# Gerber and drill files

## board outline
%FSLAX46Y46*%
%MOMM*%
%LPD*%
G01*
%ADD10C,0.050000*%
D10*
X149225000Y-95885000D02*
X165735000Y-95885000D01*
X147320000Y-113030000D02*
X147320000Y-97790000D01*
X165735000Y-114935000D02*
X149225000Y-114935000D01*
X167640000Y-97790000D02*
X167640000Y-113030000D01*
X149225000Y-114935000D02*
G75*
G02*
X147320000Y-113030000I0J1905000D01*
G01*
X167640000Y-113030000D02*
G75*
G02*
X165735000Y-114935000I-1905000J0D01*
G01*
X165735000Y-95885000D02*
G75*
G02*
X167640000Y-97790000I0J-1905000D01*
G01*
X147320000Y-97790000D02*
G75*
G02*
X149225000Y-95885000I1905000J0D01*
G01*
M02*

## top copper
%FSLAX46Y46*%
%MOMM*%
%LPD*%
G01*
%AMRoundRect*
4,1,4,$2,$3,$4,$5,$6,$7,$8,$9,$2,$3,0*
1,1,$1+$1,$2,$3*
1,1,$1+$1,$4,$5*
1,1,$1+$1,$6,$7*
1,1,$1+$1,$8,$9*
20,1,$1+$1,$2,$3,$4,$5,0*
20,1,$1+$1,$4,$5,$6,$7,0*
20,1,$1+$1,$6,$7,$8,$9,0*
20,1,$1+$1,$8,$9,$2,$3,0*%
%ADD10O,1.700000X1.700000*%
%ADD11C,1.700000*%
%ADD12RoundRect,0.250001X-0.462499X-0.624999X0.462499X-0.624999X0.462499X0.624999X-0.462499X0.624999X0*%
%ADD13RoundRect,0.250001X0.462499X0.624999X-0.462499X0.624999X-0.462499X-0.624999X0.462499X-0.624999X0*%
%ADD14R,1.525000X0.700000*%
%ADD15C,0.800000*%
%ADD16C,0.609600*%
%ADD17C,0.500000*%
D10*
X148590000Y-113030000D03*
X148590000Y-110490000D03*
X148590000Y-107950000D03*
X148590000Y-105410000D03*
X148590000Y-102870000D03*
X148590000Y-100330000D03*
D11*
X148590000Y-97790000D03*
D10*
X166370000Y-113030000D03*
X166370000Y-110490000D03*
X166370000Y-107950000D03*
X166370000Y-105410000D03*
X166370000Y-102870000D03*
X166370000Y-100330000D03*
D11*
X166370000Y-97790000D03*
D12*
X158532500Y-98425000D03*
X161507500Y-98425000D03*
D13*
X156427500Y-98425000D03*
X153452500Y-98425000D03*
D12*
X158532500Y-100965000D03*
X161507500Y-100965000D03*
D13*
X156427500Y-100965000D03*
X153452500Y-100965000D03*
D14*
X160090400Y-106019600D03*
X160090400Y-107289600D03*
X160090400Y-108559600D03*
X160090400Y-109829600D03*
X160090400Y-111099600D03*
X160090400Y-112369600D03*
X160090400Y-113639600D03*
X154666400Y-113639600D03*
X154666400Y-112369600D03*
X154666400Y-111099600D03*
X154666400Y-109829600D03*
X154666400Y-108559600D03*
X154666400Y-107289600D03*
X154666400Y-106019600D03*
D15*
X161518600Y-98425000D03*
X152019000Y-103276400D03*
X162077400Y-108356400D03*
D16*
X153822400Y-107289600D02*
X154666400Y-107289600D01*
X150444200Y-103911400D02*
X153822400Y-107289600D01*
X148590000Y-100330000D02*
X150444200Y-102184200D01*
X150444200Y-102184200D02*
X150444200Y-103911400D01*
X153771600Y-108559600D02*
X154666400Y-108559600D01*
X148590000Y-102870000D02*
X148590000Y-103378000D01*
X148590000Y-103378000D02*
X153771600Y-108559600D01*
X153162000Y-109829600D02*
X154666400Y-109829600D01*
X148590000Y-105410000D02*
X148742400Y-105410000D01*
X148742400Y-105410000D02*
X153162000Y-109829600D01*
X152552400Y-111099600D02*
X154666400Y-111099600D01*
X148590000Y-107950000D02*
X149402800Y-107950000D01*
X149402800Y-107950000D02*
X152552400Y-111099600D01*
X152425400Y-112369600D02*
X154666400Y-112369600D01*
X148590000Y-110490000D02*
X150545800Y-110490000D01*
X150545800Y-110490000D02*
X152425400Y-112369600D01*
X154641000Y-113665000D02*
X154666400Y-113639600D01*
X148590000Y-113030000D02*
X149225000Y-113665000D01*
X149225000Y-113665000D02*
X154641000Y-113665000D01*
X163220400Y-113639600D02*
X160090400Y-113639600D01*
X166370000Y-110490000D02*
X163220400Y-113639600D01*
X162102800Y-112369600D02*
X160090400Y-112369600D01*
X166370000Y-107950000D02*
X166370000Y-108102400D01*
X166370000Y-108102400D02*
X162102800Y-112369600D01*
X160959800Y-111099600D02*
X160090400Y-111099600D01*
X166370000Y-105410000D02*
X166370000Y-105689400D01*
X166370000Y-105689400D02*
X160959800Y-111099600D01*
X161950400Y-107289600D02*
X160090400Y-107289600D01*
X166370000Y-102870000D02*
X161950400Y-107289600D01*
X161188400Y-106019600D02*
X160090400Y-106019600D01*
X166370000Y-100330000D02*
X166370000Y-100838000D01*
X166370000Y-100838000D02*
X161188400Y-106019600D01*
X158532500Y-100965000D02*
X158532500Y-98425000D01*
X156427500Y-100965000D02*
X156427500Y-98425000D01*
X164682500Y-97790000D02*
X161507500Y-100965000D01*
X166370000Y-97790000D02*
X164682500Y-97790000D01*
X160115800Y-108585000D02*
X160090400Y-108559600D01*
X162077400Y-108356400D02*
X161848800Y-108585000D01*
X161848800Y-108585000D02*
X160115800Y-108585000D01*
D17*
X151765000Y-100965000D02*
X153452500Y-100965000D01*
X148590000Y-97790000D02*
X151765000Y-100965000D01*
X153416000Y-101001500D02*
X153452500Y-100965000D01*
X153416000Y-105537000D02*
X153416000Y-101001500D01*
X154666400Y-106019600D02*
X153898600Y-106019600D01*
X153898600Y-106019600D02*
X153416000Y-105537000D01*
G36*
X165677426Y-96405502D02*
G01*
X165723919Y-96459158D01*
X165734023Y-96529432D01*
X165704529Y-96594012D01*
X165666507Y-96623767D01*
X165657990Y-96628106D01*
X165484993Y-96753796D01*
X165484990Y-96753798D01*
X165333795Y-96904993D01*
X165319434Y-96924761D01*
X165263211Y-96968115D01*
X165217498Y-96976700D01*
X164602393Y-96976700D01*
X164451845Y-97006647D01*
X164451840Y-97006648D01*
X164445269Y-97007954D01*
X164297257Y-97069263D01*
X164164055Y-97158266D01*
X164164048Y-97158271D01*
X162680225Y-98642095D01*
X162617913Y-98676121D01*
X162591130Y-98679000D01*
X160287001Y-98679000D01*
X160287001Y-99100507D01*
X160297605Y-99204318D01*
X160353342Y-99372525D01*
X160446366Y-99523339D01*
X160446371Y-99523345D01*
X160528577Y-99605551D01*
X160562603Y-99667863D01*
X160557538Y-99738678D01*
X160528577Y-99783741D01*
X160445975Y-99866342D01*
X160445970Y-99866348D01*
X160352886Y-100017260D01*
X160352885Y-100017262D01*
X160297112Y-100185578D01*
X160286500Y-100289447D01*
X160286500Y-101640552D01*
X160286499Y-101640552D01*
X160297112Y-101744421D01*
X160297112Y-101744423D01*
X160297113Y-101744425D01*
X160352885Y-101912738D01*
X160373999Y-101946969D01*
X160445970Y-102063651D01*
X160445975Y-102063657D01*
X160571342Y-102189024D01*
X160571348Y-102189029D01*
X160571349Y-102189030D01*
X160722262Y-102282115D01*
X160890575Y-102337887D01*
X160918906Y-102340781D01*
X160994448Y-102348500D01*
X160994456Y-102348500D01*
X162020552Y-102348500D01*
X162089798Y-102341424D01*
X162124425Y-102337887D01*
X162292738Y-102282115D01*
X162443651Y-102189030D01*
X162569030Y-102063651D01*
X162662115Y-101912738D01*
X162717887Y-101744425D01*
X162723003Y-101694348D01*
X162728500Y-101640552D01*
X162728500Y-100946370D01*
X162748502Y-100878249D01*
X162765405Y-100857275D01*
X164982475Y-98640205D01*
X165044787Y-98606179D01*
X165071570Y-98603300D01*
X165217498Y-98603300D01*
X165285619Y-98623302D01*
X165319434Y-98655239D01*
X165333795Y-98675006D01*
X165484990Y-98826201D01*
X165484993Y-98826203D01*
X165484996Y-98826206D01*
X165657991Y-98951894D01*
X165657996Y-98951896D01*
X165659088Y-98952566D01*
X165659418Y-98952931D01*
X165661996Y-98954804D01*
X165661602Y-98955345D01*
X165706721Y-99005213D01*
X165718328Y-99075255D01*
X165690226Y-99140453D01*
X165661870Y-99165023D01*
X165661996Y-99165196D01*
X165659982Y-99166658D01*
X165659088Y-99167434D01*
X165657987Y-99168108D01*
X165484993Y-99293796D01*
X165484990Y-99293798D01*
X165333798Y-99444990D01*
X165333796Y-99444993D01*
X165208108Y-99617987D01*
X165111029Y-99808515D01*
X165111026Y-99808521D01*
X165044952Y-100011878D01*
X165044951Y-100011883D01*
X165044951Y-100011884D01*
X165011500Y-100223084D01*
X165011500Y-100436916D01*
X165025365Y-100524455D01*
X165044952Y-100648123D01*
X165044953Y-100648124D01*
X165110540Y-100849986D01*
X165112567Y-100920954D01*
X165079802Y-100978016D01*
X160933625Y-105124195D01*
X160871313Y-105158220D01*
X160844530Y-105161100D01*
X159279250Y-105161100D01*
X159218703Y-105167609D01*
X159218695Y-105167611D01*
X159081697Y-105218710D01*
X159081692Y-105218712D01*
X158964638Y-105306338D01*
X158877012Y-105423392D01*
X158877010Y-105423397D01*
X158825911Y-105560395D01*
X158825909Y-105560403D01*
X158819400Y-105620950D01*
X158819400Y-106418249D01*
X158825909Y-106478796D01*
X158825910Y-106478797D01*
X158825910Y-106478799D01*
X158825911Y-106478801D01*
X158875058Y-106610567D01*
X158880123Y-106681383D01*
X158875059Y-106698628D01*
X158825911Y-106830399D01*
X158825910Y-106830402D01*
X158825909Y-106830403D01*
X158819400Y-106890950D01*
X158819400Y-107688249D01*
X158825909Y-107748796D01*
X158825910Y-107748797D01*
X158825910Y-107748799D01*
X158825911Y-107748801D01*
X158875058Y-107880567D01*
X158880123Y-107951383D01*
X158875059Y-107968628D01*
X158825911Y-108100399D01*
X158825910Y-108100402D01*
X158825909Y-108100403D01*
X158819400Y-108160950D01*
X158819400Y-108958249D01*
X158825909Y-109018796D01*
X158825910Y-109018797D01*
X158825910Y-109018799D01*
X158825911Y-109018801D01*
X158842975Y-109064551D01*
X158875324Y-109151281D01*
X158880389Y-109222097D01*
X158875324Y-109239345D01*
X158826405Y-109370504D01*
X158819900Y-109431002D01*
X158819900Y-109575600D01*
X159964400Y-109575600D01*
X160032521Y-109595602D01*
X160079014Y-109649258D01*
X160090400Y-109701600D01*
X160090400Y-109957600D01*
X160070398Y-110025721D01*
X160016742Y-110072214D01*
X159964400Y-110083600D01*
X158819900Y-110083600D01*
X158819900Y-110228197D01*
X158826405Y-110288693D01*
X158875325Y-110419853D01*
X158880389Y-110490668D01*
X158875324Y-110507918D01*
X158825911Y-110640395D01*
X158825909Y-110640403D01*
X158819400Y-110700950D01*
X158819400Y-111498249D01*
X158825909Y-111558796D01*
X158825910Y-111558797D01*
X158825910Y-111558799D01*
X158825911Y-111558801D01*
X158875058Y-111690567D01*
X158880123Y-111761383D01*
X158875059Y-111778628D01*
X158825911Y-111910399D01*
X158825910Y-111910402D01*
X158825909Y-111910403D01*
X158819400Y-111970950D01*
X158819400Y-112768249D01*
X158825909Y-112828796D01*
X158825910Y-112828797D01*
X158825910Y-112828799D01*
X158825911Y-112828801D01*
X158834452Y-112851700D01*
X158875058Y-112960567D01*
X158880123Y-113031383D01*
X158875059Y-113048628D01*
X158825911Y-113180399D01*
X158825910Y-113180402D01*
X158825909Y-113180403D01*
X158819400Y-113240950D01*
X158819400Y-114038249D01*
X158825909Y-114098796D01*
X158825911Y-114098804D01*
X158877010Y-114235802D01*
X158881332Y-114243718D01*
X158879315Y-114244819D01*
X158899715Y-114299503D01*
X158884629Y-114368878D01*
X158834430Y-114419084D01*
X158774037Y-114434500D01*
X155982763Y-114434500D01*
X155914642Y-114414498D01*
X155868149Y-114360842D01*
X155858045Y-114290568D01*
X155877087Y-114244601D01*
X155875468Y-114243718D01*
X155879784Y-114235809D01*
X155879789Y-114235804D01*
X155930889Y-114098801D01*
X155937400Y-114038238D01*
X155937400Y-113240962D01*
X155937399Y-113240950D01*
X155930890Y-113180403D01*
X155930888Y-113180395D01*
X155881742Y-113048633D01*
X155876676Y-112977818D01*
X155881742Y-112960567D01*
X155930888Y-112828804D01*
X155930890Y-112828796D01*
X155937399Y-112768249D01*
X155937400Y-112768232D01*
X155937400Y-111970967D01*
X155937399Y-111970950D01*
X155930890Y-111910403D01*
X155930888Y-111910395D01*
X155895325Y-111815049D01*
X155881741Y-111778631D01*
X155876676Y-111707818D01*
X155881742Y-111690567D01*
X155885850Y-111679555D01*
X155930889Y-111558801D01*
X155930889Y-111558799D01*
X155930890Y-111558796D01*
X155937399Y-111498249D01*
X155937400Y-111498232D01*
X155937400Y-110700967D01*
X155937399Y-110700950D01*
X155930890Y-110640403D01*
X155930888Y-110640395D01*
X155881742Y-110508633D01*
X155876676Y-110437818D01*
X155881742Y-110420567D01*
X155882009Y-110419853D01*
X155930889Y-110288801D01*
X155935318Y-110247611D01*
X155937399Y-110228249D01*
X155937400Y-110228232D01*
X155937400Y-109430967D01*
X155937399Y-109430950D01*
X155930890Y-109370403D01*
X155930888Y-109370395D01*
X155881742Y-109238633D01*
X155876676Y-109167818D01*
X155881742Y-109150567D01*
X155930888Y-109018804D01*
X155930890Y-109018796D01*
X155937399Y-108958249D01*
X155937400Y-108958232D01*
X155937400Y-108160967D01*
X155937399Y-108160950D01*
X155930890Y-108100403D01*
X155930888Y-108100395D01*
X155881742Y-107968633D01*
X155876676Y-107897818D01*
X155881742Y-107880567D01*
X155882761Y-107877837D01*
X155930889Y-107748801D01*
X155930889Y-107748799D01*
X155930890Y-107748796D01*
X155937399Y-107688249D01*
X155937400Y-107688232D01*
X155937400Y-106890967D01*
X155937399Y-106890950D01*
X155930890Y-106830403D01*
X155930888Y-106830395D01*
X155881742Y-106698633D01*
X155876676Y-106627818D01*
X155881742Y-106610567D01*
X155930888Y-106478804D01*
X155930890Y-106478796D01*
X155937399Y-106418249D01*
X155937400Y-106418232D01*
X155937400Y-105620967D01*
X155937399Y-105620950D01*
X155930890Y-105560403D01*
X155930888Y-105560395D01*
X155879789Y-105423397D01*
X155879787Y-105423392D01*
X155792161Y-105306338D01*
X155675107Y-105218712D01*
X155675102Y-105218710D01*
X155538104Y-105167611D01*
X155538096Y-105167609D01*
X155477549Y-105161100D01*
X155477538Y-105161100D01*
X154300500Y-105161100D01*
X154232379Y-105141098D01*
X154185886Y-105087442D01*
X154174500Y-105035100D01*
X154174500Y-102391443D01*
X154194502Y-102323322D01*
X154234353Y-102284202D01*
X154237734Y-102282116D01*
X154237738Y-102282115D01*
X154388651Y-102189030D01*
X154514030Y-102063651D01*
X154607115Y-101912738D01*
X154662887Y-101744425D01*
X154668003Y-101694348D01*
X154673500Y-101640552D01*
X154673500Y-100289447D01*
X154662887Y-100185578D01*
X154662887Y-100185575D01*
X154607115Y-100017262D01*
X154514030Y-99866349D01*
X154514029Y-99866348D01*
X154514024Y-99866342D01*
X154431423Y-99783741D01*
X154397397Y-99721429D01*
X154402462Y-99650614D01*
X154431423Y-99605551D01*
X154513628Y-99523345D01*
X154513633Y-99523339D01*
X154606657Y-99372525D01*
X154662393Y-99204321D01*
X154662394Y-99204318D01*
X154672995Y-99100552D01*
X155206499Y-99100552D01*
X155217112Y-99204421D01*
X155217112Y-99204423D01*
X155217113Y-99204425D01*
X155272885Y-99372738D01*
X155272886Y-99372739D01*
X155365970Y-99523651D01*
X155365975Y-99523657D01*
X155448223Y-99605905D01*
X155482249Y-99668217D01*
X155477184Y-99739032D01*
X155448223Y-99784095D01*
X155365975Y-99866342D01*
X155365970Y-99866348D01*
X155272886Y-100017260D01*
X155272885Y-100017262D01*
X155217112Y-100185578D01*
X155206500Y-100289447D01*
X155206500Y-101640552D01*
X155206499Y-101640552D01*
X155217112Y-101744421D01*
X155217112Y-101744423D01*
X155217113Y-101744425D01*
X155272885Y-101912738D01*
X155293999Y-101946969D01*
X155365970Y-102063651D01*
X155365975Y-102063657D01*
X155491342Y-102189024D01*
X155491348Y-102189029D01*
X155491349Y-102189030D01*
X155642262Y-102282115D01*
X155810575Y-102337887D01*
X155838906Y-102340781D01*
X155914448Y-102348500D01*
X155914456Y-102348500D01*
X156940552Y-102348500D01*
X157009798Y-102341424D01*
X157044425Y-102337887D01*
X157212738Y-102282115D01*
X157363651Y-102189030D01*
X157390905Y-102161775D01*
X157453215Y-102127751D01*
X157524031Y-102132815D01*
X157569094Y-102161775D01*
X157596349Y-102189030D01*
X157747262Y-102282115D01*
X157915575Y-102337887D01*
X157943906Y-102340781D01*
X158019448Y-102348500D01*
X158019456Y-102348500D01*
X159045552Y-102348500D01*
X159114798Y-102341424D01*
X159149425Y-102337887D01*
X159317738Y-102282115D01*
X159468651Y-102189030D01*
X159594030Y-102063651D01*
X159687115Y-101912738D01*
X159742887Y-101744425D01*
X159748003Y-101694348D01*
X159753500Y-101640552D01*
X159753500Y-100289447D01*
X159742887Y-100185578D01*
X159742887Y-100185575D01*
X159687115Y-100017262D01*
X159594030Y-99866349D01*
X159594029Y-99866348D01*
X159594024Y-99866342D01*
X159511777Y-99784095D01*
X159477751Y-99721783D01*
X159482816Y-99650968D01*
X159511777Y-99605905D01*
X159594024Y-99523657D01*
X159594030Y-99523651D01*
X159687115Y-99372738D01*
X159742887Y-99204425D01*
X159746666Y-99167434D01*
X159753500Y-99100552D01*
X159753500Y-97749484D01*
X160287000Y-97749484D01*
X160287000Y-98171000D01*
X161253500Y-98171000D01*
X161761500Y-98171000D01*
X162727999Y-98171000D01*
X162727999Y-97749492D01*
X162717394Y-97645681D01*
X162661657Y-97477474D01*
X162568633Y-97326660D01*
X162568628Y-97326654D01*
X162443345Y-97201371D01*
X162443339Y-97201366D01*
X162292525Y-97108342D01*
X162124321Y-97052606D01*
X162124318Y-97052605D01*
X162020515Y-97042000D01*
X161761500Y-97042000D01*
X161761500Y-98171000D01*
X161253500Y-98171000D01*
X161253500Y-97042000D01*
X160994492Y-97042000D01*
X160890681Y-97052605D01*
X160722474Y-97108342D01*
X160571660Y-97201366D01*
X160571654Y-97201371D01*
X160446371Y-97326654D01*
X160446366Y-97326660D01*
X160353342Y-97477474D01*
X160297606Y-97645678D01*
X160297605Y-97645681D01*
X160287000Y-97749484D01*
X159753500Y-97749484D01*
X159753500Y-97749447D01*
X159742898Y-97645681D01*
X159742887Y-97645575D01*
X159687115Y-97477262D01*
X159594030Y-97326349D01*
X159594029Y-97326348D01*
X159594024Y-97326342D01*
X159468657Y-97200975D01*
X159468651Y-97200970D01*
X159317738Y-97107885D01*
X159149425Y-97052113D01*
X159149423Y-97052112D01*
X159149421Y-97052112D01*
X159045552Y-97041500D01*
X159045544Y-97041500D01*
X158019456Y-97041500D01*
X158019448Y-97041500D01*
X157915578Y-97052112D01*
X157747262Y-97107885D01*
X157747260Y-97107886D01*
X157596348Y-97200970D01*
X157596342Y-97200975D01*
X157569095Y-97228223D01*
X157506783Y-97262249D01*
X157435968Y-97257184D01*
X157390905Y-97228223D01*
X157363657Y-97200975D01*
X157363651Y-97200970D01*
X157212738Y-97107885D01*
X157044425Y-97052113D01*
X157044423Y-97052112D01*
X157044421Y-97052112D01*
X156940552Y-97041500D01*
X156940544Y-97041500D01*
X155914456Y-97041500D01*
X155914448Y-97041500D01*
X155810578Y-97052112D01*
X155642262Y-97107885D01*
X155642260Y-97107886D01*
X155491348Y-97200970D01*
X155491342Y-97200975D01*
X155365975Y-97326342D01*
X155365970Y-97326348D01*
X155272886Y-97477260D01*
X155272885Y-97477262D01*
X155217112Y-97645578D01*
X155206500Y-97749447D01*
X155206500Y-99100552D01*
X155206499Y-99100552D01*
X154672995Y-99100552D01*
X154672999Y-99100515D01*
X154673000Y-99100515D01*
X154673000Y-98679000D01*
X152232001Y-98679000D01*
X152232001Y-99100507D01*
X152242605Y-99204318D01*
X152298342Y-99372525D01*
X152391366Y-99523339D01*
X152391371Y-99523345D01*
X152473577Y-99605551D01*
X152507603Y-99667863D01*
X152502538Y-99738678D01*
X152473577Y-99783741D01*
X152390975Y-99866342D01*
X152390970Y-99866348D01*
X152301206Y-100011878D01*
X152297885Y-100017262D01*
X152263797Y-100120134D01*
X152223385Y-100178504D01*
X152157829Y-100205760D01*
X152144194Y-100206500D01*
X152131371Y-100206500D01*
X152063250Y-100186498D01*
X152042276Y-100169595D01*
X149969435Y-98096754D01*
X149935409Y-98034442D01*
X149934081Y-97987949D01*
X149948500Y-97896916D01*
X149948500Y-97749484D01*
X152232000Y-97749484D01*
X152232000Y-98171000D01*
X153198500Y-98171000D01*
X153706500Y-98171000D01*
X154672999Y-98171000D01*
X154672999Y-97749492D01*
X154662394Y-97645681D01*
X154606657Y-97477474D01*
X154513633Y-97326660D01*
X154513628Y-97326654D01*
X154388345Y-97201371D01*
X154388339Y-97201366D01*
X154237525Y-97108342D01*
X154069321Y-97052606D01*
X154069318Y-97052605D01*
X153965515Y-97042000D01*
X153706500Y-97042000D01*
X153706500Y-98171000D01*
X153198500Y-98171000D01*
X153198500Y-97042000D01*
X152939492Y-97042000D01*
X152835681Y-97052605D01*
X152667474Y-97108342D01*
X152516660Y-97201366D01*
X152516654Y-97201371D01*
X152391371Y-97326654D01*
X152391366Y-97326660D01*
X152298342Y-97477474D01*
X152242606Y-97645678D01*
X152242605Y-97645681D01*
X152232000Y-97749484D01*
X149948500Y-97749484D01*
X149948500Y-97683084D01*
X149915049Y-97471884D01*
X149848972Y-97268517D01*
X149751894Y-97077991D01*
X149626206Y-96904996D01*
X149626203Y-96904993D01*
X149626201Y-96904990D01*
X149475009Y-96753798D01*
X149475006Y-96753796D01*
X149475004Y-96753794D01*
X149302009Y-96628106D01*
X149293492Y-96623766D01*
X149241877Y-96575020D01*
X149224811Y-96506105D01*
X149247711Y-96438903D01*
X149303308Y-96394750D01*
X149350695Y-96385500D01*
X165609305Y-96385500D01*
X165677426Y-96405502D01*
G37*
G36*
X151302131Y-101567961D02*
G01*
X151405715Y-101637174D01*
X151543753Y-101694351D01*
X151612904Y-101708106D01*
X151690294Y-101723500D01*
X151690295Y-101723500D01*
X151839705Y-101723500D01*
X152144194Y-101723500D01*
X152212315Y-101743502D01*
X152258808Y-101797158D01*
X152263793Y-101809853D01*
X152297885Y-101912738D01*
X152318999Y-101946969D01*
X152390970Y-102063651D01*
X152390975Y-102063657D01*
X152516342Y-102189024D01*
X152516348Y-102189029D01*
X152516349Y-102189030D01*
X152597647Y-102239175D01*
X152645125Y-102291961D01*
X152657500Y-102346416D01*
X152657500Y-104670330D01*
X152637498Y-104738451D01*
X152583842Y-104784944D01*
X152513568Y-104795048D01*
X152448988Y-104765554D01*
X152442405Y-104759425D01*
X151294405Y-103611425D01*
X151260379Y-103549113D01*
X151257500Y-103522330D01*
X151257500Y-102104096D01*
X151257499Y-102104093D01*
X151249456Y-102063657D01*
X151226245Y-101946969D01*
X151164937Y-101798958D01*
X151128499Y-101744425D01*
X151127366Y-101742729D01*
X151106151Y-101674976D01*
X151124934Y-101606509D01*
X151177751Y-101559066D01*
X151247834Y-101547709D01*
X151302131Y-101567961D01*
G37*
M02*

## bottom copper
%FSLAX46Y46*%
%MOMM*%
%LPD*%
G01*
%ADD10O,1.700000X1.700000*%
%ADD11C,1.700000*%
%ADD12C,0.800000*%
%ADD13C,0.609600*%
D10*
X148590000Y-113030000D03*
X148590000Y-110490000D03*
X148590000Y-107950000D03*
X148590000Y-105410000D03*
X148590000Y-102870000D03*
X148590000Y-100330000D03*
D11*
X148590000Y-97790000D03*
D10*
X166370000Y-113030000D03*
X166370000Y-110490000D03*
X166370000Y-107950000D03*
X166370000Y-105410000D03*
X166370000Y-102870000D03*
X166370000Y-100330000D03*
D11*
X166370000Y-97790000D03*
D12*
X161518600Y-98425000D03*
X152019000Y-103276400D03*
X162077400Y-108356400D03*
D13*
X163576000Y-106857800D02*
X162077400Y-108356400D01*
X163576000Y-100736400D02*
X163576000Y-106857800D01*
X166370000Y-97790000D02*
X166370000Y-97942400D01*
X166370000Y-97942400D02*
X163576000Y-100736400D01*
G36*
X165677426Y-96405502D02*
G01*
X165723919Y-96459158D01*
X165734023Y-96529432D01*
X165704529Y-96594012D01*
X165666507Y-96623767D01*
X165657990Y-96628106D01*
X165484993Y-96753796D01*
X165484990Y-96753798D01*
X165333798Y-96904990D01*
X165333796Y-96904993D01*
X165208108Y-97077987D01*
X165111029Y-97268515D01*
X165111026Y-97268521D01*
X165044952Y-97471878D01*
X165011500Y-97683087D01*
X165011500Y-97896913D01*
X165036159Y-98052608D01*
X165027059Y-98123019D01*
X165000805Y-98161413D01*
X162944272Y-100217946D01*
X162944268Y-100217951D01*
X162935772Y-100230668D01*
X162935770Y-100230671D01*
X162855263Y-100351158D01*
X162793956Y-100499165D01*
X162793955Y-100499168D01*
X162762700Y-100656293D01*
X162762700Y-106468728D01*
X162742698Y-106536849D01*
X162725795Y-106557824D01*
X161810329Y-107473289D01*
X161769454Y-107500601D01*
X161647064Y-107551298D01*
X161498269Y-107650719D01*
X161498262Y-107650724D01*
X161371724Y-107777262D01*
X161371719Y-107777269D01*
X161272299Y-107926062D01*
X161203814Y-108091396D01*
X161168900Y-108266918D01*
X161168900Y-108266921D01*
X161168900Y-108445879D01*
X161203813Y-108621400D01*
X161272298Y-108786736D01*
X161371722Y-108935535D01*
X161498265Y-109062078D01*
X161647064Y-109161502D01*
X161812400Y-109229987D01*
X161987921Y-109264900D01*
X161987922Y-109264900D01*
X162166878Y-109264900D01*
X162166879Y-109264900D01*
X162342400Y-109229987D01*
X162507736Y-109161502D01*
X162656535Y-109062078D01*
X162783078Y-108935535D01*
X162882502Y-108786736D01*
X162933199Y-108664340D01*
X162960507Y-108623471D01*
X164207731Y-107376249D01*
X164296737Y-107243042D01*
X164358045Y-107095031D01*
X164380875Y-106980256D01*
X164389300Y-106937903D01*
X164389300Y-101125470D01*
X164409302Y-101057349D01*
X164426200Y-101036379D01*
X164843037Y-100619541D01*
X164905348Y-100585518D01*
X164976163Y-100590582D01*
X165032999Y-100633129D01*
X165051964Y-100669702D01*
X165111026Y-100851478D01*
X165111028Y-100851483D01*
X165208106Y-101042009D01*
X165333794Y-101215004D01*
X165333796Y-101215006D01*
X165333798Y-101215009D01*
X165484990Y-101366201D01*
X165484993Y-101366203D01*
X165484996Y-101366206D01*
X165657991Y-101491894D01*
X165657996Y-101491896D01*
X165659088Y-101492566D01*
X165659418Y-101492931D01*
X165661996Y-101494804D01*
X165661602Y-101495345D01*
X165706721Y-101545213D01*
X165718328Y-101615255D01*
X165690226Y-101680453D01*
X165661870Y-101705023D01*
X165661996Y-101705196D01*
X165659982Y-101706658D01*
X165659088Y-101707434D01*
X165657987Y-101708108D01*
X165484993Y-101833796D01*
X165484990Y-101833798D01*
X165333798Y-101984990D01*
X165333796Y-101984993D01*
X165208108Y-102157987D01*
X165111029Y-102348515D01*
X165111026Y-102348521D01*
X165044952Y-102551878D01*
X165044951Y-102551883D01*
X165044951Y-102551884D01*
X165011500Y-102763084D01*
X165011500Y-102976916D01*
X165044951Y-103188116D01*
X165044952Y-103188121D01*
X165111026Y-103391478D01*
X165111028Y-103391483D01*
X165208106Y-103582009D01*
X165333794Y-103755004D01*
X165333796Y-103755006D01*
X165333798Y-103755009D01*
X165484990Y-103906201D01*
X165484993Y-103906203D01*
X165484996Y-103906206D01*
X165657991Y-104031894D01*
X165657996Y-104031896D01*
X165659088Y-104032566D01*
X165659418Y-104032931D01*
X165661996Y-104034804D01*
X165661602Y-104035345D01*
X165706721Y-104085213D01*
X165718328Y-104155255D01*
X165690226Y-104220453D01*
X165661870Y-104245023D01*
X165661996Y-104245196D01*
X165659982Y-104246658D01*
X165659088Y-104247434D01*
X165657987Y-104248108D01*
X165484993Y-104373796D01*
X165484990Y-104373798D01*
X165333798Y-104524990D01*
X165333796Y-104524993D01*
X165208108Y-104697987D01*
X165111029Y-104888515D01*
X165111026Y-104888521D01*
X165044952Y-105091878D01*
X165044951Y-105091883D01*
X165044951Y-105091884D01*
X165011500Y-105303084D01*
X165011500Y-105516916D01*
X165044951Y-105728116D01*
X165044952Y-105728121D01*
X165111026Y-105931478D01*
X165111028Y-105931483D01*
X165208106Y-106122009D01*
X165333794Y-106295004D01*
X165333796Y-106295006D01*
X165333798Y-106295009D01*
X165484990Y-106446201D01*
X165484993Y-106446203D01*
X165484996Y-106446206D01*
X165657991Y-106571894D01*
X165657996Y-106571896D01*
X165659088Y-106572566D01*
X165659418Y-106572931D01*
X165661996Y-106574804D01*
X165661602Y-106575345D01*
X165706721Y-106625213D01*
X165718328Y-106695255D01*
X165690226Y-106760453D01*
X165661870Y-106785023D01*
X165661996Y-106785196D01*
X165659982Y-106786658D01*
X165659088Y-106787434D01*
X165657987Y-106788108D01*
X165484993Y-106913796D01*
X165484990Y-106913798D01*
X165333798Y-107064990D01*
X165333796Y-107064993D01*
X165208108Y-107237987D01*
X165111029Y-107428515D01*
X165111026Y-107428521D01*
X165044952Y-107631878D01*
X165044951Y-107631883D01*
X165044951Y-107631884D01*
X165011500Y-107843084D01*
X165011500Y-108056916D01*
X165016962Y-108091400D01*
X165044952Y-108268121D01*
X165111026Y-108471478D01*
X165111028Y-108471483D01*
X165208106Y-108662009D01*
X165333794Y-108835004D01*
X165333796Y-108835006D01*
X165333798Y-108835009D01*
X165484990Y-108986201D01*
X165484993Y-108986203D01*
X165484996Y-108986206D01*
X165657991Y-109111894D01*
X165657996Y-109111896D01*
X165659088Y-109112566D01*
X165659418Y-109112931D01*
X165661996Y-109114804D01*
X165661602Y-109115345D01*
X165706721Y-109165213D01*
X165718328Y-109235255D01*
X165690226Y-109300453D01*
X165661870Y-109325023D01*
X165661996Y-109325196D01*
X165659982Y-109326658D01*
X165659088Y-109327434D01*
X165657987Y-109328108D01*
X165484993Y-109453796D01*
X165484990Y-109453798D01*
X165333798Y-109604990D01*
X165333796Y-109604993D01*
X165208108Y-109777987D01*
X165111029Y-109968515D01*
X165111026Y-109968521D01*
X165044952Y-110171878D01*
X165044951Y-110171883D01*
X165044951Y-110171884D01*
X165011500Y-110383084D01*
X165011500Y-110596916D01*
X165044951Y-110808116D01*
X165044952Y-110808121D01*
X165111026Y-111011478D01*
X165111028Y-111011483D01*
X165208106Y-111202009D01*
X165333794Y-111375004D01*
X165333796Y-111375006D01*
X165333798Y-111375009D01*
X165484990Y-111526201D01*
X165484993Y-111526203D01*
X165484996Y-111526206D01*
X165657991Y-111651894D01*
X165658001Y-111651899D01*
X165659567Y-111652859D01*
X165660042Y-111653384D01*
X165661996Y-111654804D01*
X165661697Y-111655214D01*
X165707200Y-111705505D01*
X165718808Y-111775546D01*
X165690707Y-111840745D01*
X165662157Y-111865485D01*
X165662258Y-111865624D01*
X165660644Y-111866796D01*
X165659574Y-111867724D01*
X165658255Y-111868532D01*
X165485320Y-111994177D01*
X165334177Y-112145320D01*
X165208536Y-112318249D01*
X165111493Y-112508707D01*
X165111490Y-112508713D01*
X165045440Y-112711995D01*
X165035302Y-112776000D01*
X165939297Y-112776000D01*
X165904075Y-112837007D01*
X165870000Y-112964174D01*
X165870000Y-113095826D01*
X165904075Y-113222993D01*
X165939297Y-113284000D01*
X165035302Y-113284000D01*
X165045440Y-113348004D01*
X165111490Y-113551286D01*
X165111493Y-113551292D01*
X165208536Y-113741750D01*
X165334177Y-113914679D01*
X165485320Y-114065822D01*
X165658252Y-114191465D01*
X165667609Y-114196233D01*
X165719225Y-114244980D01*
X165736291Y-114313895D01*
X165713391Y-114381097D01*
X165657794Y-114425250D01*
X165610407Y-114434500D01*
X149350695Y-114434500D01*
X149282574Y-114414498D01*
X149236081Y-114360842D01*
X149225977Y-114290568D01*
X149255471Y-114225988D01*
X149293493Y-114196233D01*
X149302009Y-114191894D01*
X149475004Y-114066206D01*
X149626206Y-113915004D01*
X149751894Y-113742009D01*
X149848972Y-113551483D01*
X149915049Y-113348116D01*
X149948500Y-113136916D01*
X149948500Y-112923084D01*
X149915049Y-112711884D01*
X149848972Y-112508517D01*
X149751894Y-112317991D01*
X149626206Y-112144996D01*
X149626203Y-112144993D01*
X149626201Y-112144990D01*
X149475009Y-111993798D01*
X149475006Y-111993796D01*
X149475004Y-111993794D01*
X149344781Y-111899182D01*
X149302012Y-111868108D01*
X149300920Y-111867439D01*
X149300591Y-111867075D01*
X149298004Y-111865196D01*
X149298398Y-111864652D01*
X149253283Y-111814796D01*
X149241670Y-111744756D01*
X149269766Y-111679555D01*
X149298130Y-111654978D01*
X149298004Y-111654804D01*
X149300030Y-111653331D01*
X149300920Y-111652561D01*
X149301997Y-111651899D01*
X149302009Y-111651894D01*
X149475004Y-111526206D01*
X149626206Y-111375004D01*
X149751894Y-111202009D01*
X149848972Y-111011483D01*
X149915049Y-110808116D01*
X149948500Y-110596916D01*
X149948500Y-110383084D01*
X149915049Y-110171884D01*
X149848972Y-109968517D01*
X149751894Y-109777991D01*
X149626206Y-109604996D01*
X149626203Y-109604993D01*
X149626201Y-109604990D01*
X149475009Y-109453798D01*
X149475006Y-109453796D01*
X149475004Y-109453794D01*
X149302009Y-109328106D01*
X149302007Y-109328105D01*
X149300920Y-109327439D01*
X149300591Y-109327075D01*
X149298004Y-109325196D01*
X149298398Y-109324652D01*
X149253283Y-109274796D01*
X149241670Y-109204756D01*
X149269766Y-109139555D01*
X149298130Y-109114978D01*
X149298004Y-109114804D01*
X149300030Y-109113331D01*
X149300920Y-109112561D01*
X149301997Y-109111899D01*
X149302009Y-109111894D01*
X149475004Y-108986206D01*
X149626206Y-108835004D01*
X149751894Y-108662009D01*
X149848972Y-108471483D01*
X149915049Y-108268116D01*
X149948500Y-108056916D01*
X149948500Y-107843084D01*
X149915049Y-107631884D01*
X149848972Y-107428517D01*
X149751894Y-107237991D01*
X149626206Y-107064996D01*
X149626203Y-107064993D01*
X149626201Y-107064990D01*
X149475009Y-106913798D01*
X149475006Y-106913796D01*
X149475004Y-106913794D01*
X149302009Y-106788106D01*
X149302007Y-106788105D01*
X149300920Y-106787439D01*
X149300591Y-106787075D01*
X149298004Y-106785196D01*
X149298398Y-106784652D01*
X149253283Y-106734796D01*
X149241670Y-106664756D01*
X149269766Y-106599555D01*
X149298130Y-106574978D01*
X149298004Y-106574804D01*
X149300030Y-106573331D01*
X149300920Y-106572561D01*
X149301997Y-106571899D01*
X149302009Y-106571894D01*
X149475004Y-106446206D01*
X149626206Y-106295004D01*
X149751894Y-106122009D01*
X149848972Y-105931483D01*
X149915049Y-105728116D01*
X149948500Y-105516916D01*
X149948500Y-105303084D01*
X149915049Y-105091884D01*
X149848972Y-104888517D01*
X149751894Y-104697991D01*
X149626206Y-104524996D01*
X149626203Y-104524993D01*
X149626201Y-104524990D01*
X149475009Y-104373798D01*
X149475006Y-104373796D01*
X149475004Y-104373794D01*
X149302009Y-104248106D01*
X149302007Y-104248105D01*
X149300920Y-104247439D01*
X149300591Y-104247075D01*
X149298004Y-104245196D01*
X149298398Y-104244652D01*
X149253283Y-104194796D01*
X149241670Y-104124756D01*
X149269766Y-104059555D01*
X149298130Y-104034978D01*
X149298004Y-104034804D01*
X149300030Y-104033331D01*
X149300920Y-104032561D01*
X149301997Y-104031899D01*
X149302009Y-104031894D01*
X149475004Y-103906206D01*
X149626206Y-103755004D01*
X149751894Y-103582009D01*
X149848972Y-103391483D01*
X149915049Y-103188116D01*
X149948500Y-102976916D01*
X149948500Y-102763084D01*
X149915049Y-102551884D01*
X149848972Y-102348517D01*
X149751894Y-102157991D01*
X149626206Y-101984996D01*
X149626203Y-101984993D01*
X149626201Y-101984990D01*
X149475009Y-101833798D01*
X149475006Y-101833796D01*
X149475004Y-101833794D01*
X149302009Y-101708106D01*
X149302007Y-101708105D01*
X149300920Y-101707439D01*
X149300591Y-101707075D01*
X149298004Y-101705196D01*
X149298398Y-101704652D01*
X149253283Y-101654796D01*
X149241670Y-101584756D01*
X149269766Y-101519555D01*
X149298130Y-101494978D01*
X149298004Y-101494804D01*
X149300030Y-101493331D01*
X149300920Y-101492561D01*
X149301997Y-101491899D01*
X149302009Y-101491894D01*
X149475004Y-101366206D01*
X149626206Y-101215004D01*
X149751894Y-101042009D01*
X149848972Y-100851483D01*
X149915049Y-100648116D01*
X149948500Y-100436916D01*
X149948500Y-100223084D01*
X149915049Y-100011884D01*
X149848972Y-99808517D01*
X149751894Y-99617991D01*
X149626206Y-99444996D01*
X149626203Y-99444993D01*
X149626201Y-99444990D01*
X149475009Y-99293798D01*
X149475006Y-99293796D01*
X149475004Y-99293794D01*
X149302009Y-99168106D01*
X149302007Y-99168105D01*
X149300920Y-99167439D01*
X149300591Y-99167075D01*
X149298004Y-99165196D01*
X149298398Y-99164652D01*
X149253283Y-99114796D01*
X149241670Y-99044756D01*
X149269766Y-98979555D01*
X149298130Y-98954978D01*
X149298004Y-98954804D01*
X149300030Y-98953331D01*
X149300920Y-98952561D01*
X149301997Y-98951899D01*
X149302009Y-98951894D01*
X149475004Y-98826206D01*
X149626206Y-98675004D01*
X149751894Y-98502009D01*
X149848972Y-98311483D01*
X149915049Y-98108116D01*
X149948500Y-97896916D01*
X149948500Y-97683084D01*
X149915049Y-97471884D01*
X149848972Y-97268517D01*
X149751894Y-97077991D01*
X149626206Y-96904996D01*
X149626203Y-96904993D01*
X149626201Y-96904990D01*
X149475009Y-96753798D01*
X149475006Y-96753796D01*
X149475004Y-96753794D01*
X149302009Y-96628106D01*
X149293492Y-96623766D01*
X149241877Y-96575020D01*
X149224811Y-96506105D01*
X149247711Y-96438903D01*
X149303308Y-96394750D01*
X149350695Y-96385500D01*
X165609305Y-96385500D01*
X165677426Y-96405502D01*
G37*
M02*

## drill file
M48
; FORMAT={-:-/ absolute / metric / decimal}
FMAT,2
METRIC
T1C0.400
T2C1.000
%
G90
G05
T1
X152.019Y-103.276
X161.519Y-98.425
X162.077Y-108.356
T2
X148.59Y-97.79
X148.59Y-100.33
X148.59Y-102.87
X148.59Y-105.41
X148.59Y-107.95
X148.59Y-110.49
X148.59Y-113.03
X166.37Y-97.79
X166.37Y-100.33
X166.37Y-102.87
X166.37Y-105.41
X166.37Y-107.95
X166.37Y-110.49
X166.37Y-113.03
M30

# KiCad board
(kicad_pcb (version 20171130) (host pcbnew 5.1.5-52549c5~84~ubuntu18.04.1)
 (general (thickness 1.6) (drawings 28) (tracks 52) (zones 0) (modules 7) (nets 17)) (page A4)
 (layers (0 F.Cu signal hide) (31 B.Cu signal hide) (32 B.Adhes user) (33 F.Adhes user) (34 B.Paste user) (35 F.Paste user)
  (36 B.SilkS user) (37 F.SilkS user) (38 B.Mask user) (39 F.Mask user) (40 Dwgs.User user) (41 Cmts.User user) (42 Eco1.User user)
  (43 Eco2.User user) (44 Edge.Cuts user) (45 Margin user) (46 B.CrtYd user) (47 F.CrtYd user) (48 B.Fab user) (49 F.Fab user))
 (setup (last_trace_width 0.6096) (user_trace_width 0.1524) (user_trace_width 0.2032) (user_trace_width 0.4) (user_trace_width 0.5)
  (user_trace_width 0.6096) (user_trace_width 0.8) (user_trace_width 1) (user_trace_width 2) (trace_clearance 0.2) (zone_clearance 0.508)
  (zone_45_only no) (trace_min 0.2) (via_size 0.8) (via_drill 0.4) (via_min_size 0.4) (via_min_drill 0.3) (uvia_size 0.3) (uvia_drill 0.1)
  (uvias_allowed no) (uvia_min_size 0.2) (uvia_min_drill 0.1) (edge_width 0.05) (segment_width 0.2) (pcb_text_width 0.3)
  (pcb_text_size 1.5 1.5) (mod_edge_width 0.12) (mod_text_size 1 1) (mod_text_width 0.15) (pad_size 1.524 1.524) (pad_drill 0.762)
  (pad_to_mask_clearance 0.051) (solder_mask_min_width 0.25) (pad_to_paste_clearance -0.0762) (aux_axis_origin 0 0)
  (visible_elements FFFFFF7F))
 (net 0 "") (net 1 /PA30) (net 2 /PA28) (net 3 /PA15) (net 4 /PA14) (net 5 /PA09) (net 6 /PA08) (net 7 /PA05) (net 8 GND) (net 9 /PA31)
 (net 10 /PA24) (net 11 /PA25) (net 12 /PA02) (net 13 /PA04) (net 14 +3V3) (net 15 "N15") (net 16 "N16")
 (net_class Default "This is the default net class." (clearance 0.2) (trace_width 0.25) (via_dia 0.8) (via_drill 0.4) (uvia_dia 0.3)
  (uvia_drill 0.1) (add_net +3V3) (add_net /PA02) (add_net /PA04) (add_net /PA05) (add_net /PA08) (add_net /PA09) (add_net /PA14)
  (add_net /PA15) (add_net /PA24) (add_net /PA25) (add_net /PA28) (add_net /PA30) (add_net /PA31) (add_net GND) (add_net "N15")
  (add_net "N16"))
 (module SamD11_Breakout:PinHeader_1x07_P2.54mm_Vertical (layer F.Cu) (at 148.59 97.79)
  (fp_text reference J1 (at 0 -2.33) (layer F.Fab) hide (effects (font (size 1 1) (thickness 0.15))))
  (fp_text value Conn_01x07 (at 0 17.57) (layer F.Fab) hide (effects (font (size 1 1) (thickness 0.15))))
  (pad 7 thru_hole oval (at 0 15.24) (size 1.7 1.7) (drill 1) (layers *.Cu *.Mask) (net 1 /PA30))
  (pad 6 thru_hole oval (at 0 12.7) (size 1.7 1.7) (drill 1) (layers *.Cu *.Mask) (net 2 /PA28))
  (pad 5 thru_hole oval (at 0 10.16) (size 1.7 1.7) (drill 1) (layers *.Cu *.Mask) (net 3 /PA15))
  (pad 4 thru_hole oval (at 0 7.62) (size 1.7 1.7) (drill 1) (layers *.Cu *.Mask) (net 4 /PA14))
  (pad 3 thru_hole oval (at 0 5.08) (size 1.7 1.7) (drill 1) (layers *.Cu *.Mask) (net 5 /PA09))
  (pad 2 thru_hole oval (at 0 2.54) (size 1.7 1.7) (drill 1) (layers *.Cu *.Mask) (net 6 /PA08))
  (pad 1 thru_hole circle (at 0 0) (size 1.7 1.7) (drill 1) (layers *.Cu *.Mask) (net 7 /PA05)))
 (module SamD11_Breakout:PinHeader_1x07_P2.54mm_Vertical (layer F.Cu) (at 166.37 97.79)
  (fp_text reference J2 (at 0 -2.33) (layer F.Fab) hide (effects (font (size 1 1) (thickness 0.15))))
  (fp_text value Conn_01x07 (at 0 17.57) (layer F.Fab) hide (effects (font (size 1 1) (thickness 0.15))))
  (pad 7 thru_hole oval (at 0 15.24) (size 1.7 1.7) (drill 1) (layers *.Cu *.Mask) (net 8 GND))
  (pad 6 thru_hole oval (at 0 12.7) (size 1.7 1.7) (drill 1) (layers *.Cu *.Mask) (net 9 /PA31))
  (pad 5 thru_hole oval (at 0 10.16) (size 1.7 1.7) (drill 1) (layers *.Cu *.Mask) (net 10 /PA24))
  (pad 4 thru_hole oval (at 0 7.62) (size 1.7 1.7) (drill 1) (layers *.Cu *.Mask) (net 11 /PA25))
  (pad 3 thru_hole oval (at 0 5.08) (size 1.7 1.7) (drill 1) (layers *.Cu *.Mask) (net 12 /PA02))
  (pad 2 thru_hole oval (at 0 2.54) (size 1.7 1.7) (drill 1) (layers *.Cu *.Mask) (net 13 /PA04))
  (pad 1 thru_hole circle (at 0 0) (size 1.7 1.7) (drill 1) (layers *.Cu *.Mask) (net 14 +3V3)))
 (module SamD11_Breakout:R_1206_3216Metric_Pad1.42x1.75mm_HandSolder (layer F.Cu) (at 160.02 98.425)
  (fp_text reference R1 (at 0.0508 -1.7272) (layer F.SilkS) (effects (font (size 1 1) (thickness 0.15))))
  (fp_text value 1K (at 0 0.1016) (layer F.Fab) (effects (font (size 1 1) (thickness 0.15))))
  (pad 1 smd roundrect (at -1.4875 0) (size 1.425 1.75) (layers F.Cu F.Paste F.Mask) (roundrect_rratio 0.175439) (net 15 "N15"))
  (pad 2 smd roundrect (at 1.4875 0) (size 1.425 1.75) (layers F.Cu F.Paste F.Mask) (roundrect_rratio 0.175439) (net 8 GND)))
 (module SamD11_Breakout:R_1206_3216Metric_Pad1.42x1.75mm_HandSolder (layer F.Cu) (at 154.94 98.425 180)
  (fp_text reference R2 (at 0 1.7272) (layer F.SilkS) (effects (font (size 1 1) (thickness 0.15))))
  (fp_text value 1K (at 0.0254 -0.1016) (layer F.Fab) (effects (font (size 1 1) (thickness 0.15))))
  (pad 1 smd roundrect (at -1.4875 0 180) (size 1.425 1.75) (layers F.Cu F.Paste F.Mask) (roundrect_rratio 0.175439) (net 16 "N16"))
  (pad 2 smd roundrect (at 1.4875 0 180) (size 1.425 1.75) (layers F.Cu F.Paste F.Mask) (roundrect_rratio 0.175439) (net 8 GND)))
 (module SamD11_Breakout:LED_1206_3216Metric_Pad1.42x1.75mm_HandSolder (layer F.Cu) (at 160.02 100.965)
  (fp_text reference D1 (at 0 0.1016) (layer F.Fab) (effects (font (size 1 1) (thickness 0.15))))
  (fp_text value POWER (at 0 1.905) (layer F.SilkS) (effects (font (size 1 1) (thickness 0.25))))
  (pad 1 smd roundrect (at -1.4875 0) (size 1.425 1.75) (layers F.Cu F.Paste F.Mask) (roundrect_rratio 0.175439) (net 15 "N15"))
  (pad 2 smd roundrect (at 1.4875 0) (size 1.425 1.75) (layers F.Cu F.Paste F.Mask) (roundrect_rratio 0.175439) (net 14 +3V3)))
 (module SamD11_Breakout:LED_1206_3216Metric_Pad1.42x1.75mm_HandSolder (layer F.Cu) (at 154.94 100.965 180)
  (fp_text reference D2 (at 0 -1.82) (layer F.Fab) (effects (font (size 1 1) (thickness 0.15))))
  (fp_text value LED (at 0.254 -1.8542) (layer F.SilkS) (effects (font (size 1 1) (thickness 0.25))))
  (pad 1 smd roundrect (at -1.4875 0 180) (size 1.425 1.75) (layers F.Cu F.Paste F.Mask) (roundrect_rratio 0.175439) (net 16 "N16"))
  (pad 2 smd roundrect (at 1.4875 0 180) (size 1.425 1.75) (layers F.Cu F.Paste F.Mask) (roundrect_rratio 0.175439) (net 7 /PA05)))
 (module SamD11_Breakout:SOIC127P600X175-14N (layer F.Cu) (at 157.3784 109.8296)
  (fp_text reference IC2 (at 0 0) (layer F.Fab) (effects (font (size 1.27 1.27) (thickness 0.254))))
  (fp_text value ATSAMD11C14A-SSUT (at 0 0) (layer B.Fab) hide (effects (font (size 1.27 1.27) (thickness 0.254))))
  (pad 14 smd rect (at 2.712 -3.81 90) (size 0.7 1.525) (layers F.Cu F.Paste F.Mask) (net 13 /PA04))
  (pad 13 smd rect (at 2.712 -2.54 90) (size 0.7 1.525) (layers F.Cu F.Paste F.Mask) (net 12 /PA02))
  (pad 12 smd rect (at 2.712 -1.27 90) (size 0.7 1.525) (layers F.Cu F.Paste F.Mask) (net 14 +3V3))
  (pad 11 smd rect (at 2.712 0 90) (size 0.7 1.525) (layers F.Cu F.Paste F.Mask) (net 8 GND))
  (pad 10 smd rect (at 2.712 1.27 90) (size 0.7 1.525) (layers F.Cu F.Paste F.Mask) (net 11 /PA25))
  (pad 9 smd rect (at 2.712 2.54 90) (size 0.7 1.525) (layers F.Cu F.Paste F.Mask) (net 10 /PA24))
  (pad 8 smd rect (at 2.712 3.81 90) (size 0.7 1.525) (layers F.Cu F.Paste F.Mask) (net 9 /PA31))
  (pad 7 smd rect (at -2.712 3.81 90) (size 0.7 1.525) (layers F.Cu F.Paste F.Mask) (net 1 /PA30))
  (pad 6 smd rect (at -2.712 2.54 90) (size 0.7 1.525) (layers F.Cu F.Paste F.Mask) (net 2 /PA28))
  (pad 5 smd rect (at -2.712 1.27 90) (size 0.7 1.525) (layers F.Cu F.Paste F.Mask) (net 3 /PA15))
  (pad 4 smd rect (at -2.712 0 90) (size 0.7 1.525) (layers F.Cu F.Paste F.Mask) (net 4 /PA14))
  (pad 3 smd rect (at -2.712 -1.27 90) (size 0.7 1.525) (layers F.Cu F.Paste F.Mask) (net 5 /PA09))
  (pad 2 smd rect (at -2.712 -2.54 90) (size 0.7 1.525) (layers F.Cu F.Paste F.Mask) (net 6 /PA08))
  (pad 1 smd rect (at -2.712 -3.81 90) (size 0.7 1.525) (layers F.Cu F.Paste F.Mask) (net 7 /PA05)))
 (gr_line (start 149.225 95.885) (end 165.735 95.885) (layer Edge.Cuts) (width 0.05))
 (gr_line (start 147.32 113.03) (end 147.32 97.79) (layer Edge.Cuts) (width 0.05))
 (gr_line (start 165.735 114.935) (end 149.225 114.935) (layer Edge.Cuts) (width 0.05))
 (gr_line (start 167.64 97.79) (end 167.64 113.03) (layer Edge.Cuts) (width 0.05))
 (gr_arc (start 149.225 113.03) (end 147.32 113.03) (angle -90) (layer Edge.Cuts) (width 0.05))
 (gr_arc (start 165.735 113.03) (end 165.735 114.935) (angle -90) (layer Edge.Cuts) (width 0.05))
 (gr_arc (start 165.735 97.79) (end 167.64 97.79) (angle -90) (layer Edge.Cuts) (width 0.05))
 (gr_arc (start 149.225 97.79) (end 149.225 95.885) (angle -90) (layer Edge.Cuts) (width 0.05))
 (via (at 161.5186 98.425) (size 0.8) (drill 0.4) (layers F.Cu B.Cu) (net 8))
 (via (at 152.019 103.2764) (size 0.8) (drill 0.4) (layers F.Cu B.Cu) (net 8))
 (segment (start 153.8224 107.2896) (end 154.6664 107.2896) (width 0.6096) (layer F.Cu) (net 6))
 (segment (start 150.4442 103.9114) (end 153.8224 107.2896) (width 0.6096) (layer F.Cu) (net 6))
 (segment (start 148.59 100.33) (end 150.4442 102.1842) (width 0.6096) (layer F.Cu) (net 6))
 (segment (start 150.4442 102.1842) (end 150.4442 103.9114) (width 0.6096) (layer F.Cu) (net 6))
 (segment (start 153.7716 108.5596) (end 154.6664 108.5596) (width 0.6096) (layer F.Cu) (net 5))
 (segment (start 148.59 102.87) (end 148.59 103.378) (width 0.6096) (layer F.Cu) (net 5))
 (segment (start 148.59 103.378) (end 153.7716 108.5596) (width 0.6096) (layer F.Cu) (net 5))
 (segment (start 153.162 109.8296) (end 154.6664 109.8296) (width 0.6096) (layer F.Cu) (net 4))
 (segment (start 148.59 105.41) (end 148.7424 105.41) (width 0.6096) (layer F.Cu) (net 4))
 (segment (start 148.7424 105.41) (end 153.162 109.8296) (width 0.6096) (layer F.Cu) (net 4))
 (segment (start 152.5524 111.0996) (end 154.6664 111.0996) (width 0.6096) (layer F.Cu) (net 3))
 (segment (start 148.59 107.95) (end 149.4028 107.95) (width 0.6096) (layer F.Cu) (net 3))
 (segment (start 149.4028 107.95) (end 152.5524 111.0996) (width 0.6096) (layer F.Cu) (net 3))
 (segment (start 152.4254 112.3696) (end 154.6664 112.3696) (width 0.6096) (layer F.Cu) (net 2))
 (segment (start 148.59 110.49) (end 150.5458 110.49) (width 0.6096) (layer F.Cu) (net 2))
 (segment (start 150.5458 110.49) (end 152.4254 112.3696) (width 0.6096) (layer F.Cu) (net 2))
 (segment (start 154.641 113.665) (end 154.6664 113.6396) (width 0.6096) (layer F.Cu) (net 1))
 (segment (start 148.59 113.03) (end 149.225 113.665) (width 0.6096) (layer F.Cu) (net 1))
 (segment (start 149.225 113.665) (end 154.641 113.665) (width 0.6096) (layer F.Cu) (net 1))
 (segment (start 163.2204 113.6396) (end 160.0904 113.6396) (width 0.6096) (layer F.Cu) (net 9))
 (segment (start 166.37 110.49) (end 163.2204 113.6396) (width 0.6096) (layer F.Cu) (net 9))
 (segment (start 162.1028 112.3696) (end 160.0904 112.3696) (width 0.6096) (layer F.Cu) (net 10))
 (segment (start 166.37 107.95) (end 166.37 108.1024) (width 0.6096) (layer F.Cu) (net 10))
 (segment (start 166.37 108.1024) (end 162.1028 112.3696) (width 0.6096) (layer F.Cu) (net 10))
 (segment (start 160.9598 111.0996) (end 160.0904 111.0996) (width 0.6096) (layer F.Cu) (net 11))
 (segment (start 166.37 105.41) (end 166.37 105.6894) (width 0.6096) (layer F.Cu) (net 11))
 (segment (start 166.37 105.6894) (end 160.9598 111.0996) (width 0.6096) (layer F.Cu) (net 11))
 (segment (start 161.9504 107.2896) (end 160.0904 107.2896) (width 0.6096) (layer F.Cu) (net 12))
 (segment (start 166.37 102.87) (end 161.9504 107.2896) (width 0.6096) (layer F.Cu) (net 12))
 (segment (start 161.1884 106.0196) (end 160.0904 106.0196) (width 0.6096) (layer F.Cu) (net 13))
 (segment (start 166.37 100.33) (end 166.37 100.838) (width 0.6096) (layer F.Cu) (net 13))
 (segment (start 166.37 100.838) (end 161.1884 106.0196) (width 0.6096) (layer F.Cu) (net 13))
 (segment (start 158.5325 100.965) (end 158.5325 98.425) (width 0.6096) (layer F.Cu) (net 15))
 (segment (start 156.4275 100.965) (end 156.4275 98.425) (width 0.6096) (layer F.Cu) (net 16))
 (segment (start 164.6825 97.79) (end 161.5075 100.965) (width 0.6096) (layer F.Cu) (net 14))
 (segment (start 166.37 97.79) (end 164.6825 97.79) (width 0.6096) (layer F.Cu) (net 14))
 (via (at 162.0774 108.3564) (size 0.8) (drill 0.4) (layers F.Cu B.Cu) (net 14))
 (segment (start 160.1158 108.585) (end 160.0904 108.5596) (width 0.6096) (layer F.Cu) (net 14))
 (segment (start 162.0774 108.3564) (end 161.8488 108.585) (width 0.6096) (layer F.Cu) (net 14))
 (segment (start 161.8488 108.585) (end 160.1158 108.585) (width 0.6096) (layer F.Cu) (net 14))
 (segment (start 163.576 106.8578) (end 162.0774 108.3564) (width 0.6096) (layer B.Cu) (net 14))
 (segment (start 163.576 100.7364) (end 163.576 106.8578) (width 0.6096) (layer B.Cu) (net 14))
 (segment (start 166.37 97.79) (end 166.37 97.9424) (width 0.6096) (layer B.Cu) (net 14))
 (segment (start 166.37 97.9424) (end 163.576 100.7364) (width 0.6096) (layer B.Cu) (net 14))
 (segment (start 151.765 100.965) (end 153.4525 100.965) (width 0.5) (layer F.Cu) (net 7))
 (segment (start 148.59 97.79) (end 151.765 100.965) (width 0.5) (layer F.Cu) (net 7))
 (segment (start 153.416 101.0015) (end 153.4525 100.965) (width 0.5) (layer F.Cu) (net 7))
 (segment (start 153.416 105.537) (end 153.416 101.0015) (width 0.5) (layer F.Cu) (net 7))
 (segment (start 154.6664 106.0196) (end 153.8986 106.0196) (width 0.5) (layer F.Cu) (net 7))
 (segment (start 153.8986 106.0196) (end 153.416 105.537) (width 0.5) (layer F.Cu) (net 7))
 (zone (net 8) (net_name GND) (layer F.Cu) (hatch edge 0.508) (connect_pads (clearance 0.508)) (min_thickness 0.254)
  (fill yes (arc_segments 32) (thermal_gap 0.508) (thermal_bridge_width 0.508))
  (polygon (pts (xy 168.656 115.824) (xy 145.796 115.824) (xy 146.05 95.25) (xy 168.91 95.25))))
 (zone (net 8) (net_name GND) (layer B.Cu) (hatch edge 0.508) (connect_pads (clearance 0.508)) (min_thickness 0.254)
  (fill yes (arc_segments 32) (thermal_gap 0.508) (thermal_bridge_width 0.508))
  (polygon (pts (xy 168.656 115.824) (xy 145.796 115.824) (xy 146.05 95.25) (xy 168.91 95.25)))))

